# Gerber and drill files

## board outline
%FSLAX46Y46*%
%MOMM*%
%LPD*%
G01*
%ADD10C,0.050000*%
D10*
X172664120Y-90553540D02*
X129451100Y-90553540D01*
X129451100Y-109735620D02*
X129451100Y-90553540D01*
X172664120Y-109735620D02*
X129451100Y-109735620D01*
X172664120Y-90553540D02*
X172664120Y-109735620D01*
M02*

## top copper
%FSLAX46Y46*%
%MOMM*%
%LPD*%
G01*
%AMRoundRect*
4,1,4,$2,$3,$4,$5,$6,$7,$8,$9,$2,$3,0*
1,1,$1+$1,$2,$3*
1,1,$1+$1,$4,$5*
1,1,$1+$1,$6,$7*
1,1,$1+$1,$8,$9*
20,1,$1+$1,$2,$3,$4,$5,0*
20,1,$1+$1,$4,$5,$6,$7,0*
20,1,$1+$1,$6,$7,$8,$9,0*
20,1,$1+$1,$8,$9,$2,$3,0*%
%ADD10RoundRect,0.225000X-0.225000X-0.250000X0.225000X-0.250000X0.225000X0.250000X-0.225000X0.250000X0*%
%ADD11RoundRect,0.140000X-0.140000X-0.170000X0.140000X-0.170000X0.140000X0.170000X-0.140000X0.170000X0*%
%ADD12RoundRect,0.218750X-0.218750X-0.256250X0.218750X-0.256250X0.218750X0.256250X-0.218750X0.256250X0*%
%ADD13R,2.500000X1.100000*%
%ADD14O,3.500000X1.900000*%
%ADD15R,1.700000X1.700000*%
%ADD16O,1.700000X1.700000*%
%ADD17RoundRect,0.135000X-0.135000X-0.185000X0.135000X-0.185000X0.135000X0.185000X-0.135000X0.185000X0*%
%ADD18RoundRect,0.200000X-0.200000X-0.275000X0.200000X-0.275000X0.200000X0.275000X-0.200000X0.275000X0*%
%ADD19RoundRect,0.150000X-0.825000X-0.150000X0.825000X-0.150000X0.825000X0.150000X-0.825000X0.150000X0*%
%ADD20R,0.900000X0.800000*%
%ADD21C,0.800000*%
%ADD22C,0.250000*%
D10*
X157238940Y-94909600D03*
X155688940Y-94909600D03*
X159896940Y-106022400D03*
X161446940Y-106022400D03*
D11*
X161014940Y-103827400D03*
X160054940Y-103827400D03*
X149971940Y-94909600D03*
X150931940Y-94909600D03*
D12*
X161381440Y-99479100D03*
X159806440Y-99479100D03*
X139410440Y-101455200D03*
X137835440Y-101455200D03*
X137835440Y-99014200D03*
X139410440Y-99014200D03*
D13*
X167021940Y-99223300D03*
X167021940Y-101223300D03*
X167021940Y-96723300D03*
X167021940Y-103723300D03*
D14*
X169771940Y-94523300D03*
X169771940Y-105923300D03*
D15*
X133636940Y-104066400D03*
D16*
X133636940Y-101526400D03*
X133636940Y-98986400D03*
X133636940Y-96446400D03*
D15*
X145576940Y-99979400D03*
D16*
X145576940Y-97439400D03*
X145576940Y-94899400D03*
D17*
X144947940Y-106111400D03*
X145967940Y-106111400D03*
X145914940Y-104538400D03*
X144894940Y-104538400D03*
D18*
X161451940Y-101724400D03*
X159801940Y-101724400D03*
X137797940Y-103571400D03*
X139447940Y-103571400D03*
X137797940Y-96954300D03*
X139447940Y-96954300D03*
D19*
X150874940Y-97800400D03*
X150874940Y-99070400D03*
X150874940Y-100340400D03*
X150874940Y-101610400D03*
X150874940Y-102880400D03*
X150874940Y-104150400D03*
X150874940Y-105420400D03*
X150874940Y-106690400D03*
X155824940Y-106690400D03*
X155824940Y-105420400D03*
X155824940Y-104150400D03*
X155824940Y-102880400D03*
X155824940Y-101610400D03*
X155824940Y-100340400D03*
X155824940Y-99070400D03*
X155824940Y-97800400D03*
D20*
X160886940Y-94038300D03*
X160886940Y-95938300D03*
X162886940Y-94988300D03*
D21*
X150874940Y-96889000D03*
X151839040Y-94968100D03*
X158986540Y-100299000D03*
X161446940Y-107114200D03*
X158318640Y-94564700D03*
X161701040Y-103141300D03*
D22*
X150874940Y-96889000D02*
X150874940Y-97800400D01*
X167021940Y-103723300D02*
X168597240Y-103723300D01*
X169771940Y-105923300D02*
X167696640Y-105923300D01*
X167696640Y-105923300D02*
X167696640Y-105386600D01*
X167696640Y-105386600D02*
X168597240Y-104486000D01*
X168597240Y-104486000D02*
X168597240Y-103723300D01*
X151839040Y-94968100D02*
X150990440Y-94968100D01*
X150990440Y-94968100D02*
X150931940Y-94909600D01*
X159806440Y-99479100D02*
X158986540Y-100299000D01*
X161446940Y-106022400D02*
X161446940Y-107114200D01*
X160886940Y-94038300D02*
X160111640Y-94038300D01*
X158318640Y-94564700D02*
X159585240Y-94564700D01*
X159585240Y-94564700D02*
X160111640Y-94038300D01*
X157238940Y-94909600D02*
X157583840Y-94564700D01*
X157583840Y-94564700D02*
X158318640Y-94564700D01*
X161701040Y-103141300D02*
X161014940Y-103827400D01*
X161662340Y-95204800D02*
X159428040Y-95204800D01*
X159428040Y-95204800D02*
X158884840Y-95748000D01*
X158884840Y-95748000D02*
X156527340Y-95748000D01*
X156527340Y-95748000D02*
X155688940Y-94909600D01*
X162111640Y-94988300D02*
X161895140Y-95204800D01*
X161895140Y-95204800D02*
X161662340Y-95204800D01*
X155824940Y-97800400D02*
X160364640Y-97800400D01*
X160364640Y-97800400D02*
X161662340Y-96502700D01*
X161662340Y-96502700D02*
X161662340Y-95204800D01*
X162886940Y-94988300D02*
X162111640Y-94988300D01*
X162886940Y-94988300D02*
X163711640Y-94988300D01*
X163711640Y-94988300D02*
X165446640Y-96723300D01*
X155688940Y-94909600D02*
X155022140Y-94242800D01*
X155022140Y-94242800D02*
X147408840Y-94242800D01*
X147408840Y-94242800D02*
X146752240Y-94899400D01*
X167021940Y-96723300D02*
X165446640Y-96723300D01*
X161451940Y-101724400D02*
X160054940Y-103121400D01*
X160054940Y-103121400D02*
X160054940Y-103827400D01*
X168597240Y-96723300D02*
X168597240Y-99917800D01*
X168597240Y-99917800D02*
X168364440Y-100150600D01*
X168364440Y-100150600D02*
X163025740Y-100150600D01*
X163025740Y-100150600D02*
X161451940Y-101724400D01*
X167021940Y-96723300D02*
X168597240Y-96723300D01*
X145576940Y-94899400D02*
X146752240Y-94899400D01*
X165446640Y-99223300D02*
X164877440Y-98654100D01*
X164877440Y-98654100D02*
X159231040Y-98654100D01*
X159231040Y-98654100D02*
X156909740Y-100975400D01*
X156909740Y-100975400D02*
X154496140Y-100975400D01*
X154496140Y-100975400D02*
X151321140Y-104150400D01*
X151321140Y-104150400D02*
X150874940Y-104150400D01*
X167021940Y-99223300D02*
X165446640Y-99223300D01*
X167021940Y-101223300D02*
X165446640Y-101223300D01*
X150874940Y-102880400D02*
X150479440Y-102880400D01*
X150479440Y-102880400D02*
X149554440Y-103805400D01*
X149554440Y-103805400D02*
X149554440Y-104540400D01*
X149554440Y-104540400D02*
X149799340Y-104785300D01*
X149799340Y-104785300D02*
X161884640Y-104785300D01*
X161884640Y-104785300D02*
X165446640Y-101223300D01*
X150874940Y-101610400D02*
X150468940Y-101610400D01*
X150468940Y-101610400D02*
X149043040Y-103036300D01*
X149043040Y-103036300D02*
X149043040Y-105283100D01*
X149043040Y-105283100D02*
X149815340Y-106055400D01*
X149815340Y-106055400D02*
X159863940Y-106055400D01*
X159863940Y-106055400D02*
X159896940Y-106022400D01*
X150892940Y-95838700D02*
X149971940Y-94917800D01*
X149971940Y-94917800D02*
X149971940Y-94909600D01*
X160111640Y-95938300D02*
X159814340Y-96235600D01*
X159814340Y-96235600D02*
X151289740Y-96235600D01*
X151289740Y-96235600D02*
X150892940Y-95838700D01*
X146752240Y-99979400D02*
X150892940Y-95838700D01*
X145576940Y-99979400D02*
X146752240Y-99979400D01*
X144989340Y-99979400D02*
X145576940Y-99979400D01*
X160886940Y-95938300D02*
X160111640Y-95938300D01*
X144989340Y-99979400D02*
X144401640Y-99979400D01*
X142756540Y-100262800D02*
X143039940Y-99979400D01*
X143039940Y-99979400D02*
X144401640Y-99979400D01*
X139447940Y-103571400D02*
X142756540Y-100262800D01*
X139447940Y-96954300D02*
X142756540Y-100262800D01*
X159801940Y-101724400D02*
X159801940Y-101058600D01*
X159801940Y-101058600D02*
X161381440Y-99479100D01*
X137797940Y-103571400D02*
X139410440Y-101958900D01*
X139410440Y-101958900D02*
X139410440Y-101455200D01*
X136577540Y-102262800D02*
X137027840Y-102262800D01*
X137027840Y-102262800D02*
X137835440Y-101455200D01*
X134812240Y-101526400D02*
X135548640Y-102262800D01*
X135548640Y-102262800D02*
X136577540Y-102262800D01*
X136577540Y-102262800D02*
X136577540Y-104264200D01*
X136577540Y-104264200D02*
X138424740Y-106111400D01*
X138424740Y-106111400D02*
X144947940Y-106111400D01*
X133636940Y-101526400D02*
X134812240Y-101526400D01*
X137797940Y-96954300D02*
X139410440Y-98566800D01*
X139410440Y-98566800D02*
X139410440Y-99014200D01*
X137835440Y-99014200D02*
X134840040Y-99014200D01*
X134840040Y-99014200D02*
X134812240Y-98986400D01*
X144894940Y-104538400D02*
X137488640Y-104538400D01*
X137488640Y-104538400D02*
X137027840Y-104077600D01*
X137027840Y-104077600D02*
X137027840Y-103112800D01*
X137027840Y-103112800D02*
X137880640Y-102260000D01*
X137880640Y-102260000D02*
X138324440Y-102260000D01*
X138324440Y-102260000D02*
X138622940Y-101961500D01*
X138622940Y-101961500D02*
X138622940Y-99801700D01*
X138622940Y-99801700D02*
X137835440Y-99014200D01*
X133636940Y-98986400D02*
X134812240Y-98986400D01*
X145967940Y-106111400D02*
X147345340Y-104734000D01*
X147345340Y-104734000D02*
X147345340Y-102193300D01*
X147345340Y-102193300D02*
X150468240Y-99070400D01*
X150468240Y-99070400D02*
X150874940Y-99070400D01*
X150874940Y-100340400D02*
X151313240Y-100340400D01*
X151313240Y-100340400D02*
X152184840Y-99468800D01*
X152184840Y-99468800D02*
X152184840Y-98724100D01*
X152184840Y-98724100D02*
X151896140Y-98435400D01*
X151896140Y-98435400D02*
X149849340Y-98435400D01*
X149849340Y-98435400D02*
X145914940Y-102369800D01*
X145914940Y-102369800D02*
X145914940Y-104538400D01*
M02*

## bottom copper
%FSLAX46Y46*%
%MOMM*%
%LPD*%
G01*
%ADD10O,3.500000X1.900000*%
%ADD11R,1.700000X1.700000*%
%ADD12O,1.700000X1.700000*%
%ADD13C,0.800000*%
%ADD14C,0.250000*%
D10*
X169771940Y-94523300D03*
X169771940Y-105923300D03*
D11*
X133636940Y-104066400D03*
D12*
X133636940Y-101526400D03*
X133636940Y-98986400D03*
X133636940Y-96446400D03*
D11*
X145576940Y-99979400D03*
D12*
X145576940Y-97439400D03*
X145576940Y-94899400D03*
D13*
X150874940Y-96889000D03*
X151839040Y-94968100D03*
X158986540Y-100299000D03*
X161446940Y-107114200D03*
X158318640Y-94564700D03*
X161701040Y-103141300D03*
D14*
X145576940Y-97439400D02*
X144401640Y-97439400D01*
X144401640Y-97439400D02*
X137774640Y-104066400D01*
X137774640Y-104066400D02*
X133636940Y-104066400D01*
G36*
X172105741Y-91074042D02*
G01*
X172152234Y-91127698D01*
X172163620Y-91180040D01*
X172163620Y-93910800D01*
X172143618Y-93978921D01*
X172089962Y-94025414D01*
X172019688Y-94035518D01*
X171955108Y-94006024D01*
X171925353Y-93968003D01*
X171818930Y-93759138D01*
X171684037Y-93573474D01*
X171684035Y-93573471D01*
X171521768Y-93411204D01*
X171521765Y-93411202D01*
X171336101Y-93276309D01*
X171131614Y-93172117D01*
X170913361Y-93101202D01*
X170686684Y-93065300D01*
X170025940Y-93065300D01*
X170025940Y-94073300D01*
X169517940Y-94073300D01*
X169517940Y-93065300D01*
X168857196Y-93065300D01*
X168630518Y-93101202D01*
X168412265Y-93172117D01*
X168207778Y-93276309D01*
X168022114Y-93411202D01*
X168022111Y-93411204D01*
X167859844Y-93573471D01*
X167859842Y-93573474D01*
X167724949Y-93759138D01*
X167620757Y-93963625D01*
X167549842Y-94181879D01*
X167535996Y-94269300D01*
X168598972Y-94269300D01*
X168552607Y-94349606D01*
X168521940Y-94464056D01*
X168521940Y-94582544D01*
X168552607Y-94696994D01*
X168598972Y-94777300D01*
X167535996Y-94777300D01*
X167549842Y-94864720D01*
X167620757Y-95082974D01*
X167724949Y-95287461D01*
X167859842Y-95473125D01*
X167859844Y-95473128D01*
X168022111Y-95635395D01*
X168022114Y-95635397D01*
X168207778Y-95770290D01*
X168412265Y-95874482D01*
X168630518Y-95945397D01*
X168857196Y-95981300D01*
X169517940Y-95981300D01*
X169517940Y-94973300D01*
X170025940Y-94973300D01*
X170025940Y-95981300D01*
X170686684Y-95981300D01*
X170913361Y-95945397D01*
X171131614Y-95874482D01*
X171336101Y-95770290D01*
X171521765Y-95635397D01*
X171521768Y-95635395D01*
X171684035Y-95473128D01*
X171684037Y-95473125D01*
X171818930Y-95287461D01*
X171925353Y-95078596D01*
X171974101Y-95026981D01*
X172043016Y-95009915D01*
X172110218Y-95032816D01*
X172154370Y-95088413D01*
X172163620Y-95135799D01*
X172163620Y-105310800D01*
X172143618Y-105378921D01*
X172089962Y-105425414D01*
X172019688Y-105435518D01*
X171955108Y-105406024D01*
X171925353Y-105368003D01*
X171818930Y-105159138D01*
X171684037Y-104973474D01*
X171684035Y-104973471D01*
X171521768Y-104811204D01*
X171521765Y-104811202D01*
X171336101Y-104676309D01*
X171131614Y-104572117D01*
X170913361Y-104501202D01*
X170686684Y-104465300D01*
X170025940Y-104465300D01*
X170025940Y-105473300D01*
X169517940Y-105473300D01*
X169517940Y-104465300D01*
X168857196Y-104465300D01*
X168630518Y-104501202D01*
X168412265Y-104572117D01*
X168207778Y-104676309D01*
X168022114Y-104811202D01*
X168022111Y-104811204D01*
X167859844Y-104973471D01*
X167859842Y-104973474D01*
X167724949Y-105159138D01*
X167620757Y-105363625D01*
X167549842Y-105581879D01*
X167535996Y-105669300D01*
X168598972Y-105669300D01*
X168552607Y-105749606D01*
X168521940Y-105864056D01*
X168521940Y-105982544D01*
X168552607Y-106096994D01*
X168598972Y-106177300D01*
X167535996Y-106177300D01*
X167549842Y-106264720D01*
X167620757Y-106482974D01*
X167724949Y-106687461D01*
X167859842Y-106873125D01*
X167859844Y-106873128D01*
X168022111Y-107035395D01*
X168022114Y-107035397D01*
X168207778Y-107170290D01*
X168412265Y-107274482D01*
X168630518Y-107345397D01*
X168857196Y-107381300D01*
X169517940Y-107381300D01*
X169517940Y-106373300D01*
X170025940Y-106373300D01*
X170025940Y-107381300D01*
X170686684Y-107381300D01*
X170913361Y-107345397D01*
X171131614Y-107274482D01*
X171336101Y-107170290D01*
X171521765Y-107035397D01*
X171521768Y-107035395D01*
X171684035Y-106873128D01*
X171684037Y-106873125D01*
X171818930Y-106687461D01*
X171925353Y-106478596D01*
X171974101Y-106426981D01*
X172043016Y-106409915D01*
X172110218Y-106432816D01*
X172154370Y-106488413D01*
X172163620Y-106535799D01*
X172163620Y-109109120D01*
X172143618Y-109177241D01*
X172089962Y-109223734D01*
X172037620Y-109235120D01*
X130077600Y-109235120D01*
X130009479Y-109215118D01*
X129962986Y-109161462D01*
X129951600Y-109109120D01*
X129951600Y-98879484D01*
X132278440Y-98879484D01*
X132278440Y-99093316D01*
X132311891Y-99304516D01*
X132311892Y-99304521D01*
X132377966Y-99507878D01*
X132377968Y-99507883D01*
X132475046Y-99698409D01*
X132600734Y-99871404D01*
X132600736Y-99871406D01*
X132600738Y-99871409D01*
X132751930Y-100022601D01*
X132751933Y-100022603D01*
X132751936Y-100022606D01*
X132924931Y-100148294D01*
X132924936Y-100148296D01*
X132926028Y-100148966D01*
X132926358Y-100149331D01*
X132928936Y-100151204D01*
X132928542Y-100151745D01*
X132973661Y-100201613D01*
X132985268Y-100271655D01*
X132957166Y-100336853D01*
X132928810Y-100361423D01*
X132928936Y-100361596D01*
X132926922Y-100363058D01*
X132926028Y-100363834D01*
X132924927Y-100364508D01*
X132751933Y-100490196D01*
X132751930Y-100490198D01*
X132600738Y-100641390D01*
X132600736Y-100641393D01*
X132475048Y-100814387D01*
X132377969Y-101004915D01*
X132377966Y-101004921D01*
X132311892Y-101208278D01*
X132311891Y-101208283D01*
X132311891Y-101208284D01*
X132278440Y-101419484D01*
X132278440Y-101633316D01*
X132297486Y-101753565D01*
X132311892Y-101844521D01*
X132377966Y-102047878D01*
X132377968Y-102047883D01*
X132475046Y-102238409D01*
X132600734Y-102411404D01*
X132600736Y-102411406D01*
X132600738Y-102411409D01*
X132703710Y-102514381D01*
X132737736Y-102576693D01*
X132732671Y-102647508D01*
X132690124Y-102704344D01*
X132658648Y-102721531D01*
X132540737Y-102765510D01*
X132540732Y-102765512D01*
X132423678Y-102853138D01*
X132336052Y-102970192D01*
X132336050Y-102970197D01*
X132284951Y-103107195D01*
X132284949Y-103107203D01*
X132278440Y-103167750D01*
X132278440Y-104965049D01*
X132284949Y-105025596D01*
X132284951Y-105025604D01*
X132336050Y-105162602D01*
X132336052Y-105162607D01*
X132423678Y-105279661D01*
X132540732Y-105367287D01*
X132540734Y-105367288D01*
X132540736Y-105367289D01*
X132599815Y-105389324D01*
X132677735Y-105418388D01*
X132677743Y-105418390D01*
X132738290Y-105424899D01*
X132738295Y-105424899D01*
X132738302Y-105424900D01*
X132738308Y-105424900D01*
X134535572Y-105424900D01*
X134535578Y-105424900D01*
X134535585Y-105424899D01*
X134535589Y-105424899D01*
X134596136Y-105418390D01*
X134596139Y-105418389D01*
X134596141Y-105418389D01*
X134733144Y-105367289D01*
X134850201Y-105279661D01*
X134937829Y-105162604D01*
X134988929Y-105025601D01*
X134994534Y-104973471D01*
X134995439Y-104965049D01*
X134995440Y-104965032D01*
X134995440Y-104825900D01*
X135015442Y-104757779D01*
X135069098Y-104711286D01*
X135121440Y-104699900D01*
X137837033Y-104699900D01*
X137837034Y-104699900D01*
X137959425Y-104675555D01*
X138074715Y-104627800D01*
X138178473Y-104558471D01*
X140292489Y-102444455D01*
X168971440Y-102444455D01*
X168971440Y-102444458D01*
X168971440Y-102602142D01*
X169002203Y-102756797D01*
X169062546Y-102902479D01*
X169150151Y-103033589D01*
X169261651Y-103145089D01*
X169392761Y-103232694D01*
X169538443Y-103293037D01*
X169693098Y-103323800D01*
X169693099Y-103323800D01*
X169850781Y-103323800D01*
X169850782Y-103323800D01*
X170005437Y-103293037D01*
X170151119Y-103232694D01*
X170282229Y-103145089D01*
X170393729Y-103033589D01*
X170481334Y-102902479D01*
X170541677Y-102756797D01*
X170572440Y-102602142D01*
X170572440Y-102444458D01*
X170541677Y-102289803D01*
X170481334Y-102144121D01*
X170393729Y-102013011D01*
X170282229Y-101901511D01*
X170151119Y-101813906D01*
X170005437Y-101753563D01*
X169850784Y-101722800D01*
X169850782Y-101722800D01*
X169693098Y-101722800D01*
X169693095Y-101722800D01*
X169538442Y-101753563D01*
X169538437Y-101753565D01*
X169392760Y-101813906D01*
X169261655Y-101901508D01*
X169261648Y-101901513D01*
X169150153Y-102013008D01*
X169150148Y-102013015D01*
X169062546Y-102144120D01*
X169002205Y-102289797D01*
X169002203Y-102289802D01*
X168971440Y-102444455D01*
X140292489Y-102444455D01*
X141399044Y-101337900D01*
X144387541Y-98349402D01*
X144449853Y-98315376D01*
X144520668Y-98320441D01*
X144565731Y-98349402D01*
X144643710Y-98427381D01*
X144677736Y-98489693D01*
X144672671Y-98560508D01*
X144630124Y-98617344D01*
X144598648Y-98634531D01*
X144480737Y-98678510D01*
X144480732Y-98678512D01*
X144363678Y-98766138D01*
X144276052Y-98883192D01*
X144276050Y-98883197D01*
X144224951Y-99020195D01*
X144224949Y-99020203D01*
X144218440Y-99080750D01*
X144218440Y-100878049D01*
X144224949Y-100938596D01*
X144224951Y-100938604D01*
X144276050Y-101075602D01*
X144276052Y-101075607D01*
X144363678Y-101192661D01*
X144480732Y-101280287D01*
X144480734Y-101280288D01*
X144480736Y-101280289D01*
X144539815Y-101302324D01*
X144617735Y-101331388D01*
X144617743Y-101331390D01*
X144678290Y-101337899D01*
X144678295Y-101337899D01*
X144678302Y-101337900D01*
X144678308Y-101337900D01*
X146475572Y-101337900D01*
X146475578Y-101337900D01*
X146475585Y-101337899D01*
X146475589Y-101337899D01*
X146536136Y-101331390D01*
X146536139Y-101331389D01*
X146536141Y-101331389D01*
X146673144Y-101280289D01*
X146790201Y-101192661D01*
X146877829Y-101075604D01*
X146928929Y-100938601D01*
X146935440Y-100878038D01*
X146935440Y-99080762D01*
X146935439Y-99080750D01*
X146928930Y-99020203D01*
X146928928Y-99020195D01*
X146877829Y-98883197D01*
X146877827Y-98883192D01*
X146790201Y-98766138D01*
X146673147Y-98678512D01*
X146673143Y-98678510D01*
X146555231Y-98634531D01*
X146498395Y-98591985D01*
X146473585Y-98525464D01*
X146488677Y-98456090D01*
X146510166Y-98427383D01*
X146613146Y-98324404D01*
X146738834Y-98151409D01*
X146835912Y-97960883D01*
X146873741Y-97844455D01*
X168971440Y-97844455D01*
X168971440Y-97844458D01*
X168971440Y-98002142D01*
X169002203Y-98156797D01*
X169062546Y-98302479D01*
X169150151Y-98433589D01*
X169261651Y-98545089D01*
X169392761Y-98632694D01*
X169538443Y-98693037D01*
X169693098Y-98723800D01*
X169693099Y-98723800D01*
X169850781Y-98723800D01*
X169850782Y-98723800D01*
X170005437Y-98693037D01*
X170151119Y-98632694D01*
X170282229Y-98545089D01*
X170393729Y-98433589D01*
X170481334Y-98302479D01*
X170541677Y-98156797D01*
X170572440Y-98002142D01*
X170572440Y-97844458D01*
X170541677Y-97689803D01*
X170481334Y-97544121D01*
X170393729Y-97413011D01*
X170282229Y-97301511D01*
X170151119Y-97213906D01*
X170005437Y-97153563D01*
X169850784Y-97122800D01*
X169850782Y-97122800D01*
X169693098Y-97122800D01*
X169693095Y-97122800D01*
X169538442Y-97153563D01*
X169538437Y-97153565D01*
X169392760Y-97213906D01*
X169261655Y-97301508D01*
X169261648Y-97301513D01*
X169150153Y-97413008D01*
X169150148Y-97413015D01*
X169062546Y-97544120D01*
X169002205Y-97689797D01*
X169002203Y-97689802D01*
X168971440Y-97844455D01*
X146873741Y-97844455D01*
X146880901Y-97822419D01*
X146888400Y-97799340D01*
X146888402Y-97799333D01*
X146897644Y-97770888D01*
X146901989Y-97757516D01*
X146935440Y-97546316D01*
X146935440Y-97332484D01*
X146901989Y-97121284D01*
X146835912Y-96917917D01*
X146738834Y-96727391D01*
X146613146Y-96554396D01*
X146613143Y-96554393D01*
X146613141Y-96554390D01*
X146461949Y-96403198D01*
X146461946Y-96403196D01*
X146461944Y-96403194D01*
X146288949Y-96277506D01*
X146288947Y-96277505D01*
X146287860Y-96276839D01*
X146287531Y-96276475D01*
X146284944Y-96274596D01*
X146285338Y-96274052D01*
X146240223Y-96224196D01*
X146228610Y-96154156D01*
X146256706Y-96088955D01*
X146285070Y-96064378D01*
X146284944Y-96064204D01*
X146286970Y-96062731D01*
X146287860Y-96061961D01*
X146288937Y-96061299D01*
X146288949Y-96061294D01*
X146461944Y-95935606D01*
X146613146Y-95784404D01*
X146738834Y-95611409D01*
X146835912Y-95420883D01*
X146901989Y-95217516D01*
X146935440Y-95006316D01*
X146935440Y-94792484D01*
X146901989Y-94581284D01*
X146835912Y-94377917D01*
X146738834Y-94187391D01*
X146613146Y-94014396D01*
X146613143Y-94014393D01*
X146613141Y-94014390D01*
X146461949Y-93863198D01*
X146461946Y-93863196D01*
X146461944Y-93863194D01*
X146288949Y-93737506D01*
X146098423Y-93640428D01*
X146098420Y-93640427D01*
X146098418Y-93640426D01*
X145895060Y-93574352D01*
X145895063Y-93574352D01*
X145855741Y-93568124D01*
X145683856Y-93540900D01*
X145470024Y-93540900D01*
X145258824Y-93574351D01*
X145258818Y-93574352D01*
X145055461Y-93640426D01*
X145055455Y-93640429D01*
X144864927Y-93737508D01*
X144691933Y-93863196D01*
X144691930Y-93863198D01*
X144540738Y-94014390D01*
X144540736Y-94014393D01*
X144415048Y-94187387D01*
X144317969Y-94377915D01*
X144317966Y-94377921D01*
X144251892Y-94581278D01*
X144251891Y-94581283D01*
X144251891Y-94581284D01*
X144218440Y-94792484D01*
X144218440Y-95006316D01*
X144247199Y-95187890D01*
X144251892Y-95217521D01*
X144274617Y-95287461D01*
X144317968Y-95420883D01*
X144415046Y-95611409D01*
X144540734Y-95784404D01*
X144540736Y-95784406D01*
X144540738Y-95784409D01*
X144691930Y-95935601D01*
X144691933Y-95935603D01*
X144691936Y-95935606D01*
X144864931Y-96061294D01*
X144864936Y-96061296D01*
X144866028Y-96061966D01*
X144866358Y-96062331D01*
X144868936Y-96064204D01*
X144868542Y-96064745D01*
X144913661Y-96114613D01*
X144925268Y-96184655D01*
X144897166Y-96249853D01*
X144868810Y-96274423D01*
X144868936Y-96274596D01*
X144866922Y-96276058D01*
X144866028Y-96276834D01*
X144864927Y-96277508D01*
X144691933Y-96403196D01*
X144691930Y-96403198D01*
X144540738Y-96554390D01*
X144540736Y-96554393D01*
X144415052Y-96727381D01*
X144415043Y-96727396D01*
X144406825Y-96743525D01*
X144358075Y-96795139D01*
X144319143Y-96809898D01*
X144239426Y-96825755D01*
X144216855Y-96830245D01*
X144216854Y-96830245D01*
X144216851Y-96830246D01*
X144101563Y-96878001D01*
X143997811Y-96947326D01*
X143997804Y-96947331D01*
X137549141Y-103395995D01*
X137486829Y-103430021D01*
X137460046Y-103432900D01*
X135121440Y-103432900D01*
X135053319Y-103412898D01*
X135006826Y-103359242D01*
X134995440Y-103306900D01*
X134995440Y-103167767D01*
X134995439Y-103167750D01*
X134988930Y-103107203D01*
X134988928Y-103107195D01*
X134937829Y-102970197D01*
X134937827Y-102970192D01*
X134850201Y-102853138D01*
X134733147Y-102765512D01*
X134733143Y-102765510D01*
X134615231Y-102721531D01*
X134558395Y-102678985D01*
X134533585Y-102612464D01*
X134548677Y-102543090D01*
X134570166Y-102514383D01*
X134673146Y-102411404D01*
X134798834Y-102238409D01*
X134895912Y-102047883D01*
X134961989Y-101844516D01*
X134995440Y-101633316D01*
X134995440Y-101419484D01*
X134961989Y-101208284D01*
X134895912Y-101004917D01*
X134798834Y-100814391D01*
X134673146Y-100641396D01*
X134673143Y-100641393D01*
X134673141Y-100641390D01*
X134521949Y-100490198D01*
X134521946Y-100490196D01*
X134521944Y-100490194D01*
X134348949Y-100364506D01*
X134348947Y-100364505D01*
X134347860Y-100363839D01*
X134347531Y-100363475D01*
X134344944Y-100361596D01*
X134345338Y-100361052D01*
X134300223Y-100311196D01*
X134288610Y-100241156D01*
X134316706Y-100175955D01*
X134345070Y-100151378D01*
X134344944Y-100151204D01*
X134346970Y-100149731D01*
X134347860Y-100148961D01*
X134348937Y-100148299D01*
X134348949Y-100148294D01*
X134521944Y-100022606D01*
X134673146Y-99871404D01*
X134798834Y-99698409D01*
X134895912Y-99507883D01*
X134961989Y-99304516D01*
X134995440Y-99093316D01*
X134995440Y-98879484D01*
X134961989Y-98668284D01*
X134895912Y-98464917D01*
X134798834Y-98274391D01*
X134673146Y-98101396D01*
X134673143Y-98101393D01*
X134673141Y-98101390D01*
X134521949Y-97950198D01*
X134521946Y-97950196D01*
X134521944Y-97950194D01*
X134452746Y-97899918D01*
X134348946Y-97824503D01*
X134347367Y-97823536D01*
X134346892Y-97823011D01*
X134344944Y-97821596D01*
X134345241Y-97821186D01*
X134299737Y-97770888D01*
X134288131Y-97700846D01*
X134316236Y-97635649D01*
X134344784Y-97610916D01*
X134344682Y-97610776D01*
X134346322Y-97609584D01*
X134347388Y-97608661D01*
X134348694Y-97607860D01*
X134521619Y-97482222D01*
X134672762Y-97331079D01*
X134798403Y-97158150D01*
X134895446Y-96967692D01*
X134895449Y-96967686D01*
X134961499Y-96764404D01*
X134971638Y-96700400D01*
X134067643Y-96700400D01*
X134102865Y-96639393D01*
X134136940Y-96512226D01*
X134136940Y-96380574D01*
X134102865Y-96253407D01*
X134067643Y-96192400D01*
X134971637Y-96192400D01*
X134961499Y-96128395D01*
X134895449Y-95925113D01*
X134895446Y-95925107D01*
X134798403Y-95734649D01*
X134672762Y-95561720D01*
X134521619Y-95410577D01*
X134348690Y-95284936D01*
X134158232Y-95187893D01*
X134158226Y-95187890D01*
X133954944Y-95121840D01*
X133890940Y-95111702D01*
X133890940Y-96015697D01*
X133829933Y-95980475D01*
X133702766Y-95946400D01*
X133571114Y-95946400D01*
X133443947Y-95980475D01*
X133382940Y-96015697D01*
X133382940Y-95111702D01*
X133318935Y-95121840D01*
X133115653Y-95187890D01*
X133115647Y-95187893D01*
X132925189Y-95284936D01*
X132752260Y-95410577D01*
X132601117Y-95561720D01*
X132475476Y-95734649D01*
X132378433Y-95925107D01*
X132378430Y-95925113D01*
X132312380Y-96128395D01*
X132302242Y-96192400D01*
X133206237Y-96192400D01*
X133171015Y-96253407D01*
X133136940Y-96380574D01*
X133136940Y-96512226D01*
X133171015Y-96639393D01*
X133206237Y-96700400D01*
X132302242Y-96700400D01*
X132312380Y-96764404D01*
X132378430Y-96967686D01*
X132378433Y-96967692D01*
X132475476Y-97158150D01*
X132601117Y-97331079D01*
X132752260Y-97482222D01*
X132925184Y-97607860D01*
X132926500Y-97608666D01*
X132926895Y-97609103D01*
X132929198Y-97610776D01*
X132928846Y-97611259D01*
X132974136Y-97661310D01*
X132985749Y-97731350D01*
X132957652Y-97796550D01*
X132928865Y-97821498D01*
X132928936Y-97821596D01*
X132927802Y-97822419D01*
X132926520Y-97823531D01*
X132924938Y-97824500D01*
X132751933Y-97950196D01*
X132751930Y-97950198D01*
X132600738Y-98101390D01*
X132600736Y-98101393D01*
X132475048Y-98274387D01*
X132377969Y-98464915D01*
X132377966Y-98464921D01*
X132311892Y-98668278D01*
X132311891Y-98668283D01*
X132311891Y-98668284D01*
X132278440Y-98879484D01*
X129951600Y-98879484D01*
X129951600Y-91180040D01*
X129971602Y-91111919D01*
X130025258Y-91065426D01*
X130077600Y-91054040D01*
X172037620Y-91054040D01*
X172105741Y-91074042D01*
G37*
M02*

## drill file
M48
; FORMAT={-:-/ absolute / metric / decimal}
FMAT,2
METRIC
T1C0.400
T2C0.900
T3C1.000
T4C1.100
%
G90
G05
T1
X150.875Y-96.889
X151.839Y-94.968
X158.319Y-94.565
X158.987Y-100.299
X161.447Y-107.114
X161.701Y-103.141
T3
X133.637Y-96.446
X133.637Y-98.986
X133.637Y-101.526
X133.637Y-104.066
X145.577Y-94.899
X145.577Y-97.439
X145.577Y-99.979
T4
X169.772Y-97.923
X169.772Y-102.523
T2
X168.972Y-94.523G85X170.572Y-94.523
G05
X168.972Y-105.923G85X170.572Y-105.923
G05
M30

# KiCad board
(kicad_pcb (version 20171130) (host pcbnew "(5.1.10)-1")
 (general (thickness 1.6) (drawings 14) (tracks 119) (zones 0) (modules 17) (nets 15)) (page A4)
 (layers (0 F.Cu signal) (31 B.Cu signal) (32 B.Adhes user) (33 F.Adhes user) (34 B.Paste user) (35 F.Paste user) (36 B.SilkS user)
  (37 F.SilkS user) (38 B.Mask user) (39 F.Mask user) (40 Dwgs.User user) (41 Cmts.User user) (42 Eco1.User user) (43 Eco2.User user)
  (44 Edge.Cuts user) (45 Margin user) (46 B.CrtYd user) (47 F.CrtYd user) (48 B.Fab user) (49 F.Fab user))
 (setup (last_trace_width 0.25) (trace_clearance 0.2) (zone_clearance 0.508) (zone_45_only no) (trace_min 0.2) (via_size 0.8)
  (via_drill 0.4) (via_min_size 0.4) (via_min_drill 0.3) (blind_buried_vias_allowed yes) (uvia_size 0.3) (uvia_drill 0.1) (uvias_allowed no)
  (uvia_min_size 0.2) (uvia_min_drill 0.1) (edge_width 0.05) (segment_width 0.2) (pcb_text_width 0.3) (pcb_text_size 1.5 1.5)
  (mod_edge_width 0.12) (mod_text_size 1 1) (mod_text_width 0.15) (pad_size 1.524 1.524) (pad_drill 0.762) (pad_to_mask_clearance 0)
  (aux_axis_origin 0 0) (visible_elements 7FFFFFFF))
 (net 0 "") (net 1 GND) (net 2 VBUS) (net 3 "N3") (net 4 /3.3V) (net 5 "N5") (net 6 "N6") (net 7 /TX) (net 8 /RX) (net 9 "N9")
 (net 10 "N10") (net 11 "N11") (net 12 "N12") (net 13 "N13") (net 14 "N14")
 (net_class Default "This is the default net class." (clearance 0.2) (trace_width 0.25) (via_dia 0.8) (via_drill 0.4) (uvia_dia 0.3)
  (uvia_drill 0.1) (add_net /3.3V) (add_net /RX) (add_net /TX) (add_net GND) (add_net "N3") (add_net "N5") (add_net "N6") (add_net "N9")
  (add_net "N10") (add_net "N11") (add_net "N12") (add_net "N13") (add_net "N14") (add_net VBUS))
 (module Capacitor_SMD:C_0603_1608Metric (layer F.Cu) (at 156.46394 94.9096)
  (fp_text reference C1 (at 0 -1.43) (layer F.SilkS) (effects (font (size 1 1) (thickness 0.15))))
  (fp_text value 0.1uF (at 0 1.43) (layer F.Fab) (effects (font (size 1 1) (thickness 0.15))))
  (pad 2 smd roundrect (at 0.775 0) (size 0.9 0.95) (layers F.Cu F.Paste F.Mask) (roundrect_rratio 0.25) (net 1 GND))
  (pad 1 smd roundrect (at -0.775 0) (size 0.9 0.95) (layers F.Cu F.Paste F.Mask) (roundrect_rratio 0.25) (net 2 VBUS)))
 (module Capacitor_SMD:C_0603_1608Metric (layer F.Cu) (at 160.67194 106.0224)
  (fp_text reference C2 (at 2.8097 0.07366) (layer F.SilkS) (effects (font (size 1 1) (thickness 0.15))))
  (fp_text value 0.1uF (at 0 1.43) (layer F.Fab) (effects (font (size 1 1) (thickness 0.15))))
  (pad 1 smd roundrect (at -0.775 0) (size 0.9 0.95) (layers F.Cu F.Paste F.Mask) (roundrect_rratio 0.25) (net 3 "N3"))
  (pad 2 smd roundrect (at 0.775 0) (size 0.9 0.95) (layers F.Cu F.Paste F.Mask) (roundrect_rratio 0.25) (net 1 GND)))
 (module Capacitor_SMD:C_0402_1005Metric (layer F.Cu) (at 160.53494 103.8274)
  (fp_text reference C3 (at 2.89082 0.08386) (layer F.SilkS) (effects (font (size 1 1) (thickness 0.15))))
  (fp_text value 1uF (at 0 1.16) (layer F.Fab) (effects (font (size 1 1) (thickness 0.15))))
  (pad 2 smd roundrect (at 0.48 0) (size 0.56 0.62) (layers F.Cu F.Paste F.Mask) (roundrect_rratio 0.25) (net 1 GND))
  (pad 1 smd roundrect (at -0.48 0) (size 0.56 0.62) (layers F.Cu F.Paste F.Mask) (roundrect_rratio 0.25) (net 2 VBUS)))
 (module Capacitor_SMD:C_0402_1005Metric (layer F.Cu) (at 150.45194 94.9096)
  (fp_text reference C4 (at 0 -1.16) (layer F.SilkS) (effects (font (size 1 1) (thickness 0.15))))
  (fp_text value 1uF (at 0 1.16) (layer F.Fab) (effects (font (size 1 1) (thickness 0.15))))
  (pad 1 smd roundrect (at -0.48 0) (size 0.56 0.62) (layers F.Cu F.Paste F.Mask) (roundrect_rratio 0.25) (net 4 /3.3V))
  (pad 2 smd roundrect (at 0.48 0) (size 0.56 0.62) (layers F.Cu F.Paste F.Mask) (roundrect_rratio 0.25) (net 1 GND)))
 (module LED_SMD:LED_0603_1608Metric (layer F.Cu) (at 160.59394 99.4791)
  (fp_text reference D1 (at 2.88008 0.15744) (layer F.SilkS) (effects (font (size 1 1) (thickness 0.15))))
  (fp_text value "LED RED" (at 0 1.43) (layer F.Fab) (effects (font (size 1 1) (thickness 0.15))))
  (pad 2 smd roundrect (at 0.7875 0) (size 0.875 0.95) (layers F.Cu F.Paste F.Mask) (roundrect_rratio 0.25) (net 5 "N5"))
  (pad 1 smd roundrect (at -0.7875 0) (size 0.875 0.95) (layers F.Cu F.Paste F.Mask) (roundrect_rratio 0.25) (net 1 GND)))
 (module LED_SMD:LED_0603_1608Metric (layer F.Cu) (at 138.62294 101.4552)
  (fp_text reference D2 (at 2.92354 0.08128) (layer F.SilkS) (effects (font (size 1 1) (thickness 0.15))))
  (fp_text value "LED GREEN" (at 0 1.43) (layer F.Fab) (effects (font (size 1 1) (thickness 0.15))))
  (pad 2 smd roundrect (at 0.7875 0) (size 0.875 0.95) (layers F.Cu F.Paste F.Mask) (roundrect_rratio 0.25) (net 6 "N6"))
  (pad 1 smd roundrect (at -0.7875 0) (size 0.875 0.95) (layers F.Cu F.Paste F.Mask) (roundrect_rratio 0.25) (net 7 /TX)))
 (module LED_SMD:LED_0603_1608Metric (layer F.Cu) (at 138.62294 99.0142)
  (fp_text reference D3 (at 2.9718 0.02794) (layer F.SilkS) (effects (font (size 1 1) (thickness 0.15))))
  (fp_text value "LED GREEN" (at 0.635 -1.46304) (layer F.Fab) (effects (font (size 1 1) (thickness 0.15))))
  (pad 1 smd roundrect (at -0.7875 0) (size 0.875 0.95) (layers F.Cu F.Paste F.Mask) (roundrect_rratio 0.25) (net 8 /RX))
  (pad 2 smd roundrect (at 0.7875 0) (size 0.875 0.95) (layers F.Cu F.Paste F.Mask) (roundrect_rratio 0.25) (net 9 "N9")))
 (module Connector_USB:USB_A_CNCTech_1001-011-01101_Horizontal (layer F.Cu) (at 176.67194 100.2233)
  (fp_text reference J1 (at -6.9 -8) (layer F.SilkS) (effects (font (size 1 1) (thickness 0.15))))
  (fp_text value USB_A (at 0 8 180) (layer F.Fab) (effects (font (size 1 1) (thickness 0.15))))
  (pad 2 smd rect (at -9.65 -1) (size 2.5 1.1) (layers F.Cu F.Paste F.Mask) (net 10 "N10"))
  (pad 3 smd rect (at -9.65 1) (size 2.5 1.1) (layers F.Cu F.Paste F.Mask) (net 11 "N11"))
  (pad 1 smd rect (at -9.65 -3.5) (size 2.5 1.1) (layers F.Cu F.Paste F.Mask) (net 2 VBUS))
  (pad 4 smd rect (at -9.65 3.5) (size 2.5 1.1) (layers F.Cu F.Paste F.Mask) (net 1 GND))
  (pad 5 thru_hole oval (at -6.9 -5.7) (size 3.5 1.9) (drill oval 2.5 0.9) (layers *.Cu *.Mask) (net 1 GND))
  (pad 5 thru_hole oval (at -6.9 5.7) (size 3.5 1.9) (drill oval 2.5 0.9) (layers *.Cu *.Mask) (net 1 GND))
  (pad "" np_thru_hole circle (at -6.9 -2.3) (size 1.1 1.1) (drill 1.1) (layers *.Cu *.Mask))
  (pad "" np_thru_hole circle (at -6.9 2.3) (size 1.1 1.1) (drill 1.1) (layers *.Cu *.Mask)))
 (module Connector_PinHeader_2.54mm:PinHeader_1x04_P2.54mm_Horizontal (layer F.Cu) (at 133.63694 104.0664 180)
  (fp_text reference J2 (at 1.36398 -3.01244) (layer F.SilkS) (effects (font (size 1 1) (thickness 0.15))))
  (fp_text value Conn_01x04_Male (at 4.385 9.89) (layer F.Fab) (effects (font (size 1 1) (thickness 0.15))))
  (pad 1 thru_hole rect (at 0 0 180) (size 1.7 1.7) (drill 1) (layers *.Cu *.Mask) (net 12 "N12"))
  (pad 2 thru_hole oval (at 0 2.54 180) (size 1.7 1.7) (drill 1) (layers *.Cu *.Mask) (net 7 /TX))
  (pad 3 thru_hole oval (at 0 5.08 180) (size 1.7 1.7) (drill 1) (layers *.Cu *.Mask) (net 8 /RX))
  (pad 4 thru_hole oval (at 0 7.62 180) (size 1.7 1.7) (drill 1) (layers *.Cu *.Mask) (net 1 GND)))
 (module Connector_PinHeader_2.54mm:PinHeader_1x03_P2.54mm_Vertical (layer F.Cu) (at 145.57694 99.9794 180)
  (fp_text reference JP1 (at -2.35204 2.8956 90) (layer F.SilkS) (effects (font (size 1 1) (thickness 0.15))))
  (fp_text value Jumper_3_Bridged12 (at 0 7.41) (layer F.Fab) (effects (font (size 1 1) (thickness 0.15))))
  (pad 1 thru_hole rect (at 0 0 180) (size 1.7 1.7) (drill 1) (layers *.Cu *.Mask) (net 4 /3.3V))
  (pad 2 thru_hole oval (at 0 2.54 180) (size 1.7 1.7) (drill 1) (layers *.Cu *.Mask) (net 12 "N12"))
  (pad 3 thru_hole oval (at 0 5.08 180) (size 1.7 1.7) (drill 1) (layers *.Cu *.Mask) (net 2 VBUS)))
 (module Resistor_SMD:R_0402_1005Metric (layer F.Cu) (at 145.45794 106.1114)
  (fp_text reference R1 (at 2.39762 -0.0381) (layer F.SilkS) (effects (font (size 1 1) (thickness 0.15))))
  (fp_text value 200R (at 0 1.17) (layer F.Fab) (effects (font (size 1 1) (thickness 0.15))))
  (pad 1 smd roundrect (at -0.51 0) (size 0.54 0.64) (layers F.Cu F.Paste F.Mask) (roundrect_rratio 0.25) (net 7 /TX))
  (pad 2 smd roundrect (at 0.51 0) (size 0.54 0.64) (layers F.Cu F.Paste F.Mask) (roundrect_rratio 0.25) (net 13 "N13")))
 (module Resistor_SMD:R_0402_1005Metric (layer F.Cu) (at 145.40494 104.5384)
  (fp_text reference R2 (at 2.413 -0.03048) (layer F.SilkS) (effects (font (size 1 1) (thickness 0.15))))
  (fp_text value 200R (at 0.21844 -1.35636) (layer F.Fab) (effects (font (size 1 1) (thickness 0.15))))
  (pad 2 smd roundrect (at 0.51 0) (size 0.54 0.64) (layers F.Cu F.Paste F.Mask) (roundrect_rratio 0.25) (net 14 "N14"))
  (pad 1 smd roundrect (at -0.51 0) (size 0.54 0.64) (layers F.Cu F.Paste F.Mask) (roundrect_rratio 0.25) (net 8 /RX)))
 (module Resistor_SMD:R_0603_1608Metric (layer F.Cu) (at 160.62694 101.7244)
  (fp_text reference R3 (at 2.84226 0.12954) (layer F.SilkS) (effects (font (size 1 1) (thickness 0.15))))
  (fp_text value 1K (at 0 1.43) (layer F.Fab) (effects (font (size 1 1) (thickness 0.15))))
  (pad 2 smd roundrect (at 0.825 0) (size 0.8 0.95) (layers F.Cu F.Paste F.Mask) (roundrect_rratio 0.25) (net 2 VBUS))
  (pad 1 smd roundrect (at -0.825 0) (size 0.8 0.95) (layers F.Cu F.Paste F.Mask) (roundrect_rratio 0.25) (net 5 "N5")))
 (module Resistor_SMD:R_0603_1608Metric (layer F.Cu) (at 138.62294 103.5714)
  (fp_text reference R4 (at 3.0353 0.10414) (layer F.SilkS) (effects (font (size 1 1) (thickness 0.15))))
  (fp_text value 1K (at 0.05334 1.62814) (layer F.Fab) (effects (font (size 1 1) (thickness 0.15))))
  (pad 1 smd roundrect (at -0.825 0) (size 0.8 0.95) (layers F.Cu F.Paste F.Mask) (roundrect_rratio 0.25) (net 6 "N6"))
  (pad 2 smd roundrect (at 0.825 0) (size 0.8 0.95) (layers F.Cu F.Paste F.Mask) (roundrect_rratio 0.25) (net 4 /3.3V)))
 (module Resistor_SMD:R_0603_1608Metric (layer F.Cu) (at 138.62294 96.9543)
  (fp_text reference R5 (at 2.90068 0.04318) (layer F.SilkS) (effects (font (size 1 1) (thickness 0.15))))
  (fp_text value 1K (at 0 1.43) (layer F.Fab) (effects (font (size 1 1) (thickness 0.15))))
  (pad 1 smd roundrect (at -0.825 0) (size 0.8 0.95) (layers F.Cu F.Paste F.Mask) (roundrect_rratio 0.25) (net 9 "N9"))
  (pad 2 smd roundrect (at 0.825 0) (size 0.8 0.95) (layers F.Cu F.Paste F.Mask) (roundrect_rratio 0.25) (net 4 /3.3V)))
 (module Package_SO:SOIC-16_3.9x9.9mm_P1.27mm (layer F.Cu) (at 153.34994 102.2454)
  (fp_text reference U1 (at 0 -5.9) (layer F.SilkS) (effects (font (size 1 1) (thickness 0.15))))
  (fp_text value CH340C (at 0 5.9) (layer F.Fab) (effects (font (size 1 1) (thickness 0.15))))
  (pad 1 smd roundrect (at -2.475 -4.445) (size 1.95 0.6) (layers F.Cu F.Paste F.Mask) (roundrect_rratio 0.25) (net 1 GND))
  (pad 2 smd roundrect (at -2.475 -3.175) (size 1.95 0.6) (layers F.Cu F.Paste F.Mask) (roundrect_rratio 0.25) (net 13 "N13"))
  (pad 3 smd roundrect (at -2.475 -1.905) (size 1.95 0.6) (layers F.Cu F.Paste F.Mask) (roundrect_rratio 0.25) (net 14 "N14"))
  (pad 4 smd roundrect (at -2.475 -0.635) (size 1.95 0.6) (layers F.Cu F.Paste F.Mask) (roundrect_rratio 0.25) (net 3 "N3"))
  (pad 5 smd roundrect (at -2.475 0.635) (size 1.95 0.6) (layers F.Cu F.Paste F.Mask) (roundrect_rratio 0.25) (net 11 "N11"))
  (pad 6 smd roundrect (at -2.475 1.905) (size 1.95 0.6) (layers F.Cu F.Paste F.Mask) (roundrect_rratio 0.25) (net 10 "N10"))
  (pad 7 smd roundrect (at -2.475 3.175) (size 1.95 0.6) (layers F.Cu F.Paste F.Mask) (roundrect_rratio 0.25))
  (pad 8 smd roundrect (at -2.475 4.445) (size 1.95 0.6) (layers F.Cu F.Paste F.Mask) (roundrect_rratio 0.25))
  (pad 9 smd roundrect (at 2.475 4.445) (size 1.95 0.6) (layers F.Cu F.Paste F.Mask) (roundrect_rratio 0.25))
  (pad 10 smd roundrect (at 2.475 3.175) (size 1.95 0.6) (layers F.Cu F.Paste F.Mask) (roundrect_rratio 0.25))
  (pad 11 smd roundrect (at 2.475 1.905) (size 1.95 0.6) (layers F.Cu F.Paste F.Mask) (roundrect_rratio 0.25))
  (pad 12 smd roundrect (at 2.475 0.635) (size 1.95 0.6) (layers F.Cu F.Paste F.Mask) (roundrect_rratio 0.25))
  (pad 13 smd roundrect (at 2.475 -0.635) (size 1.95 0.6) (layers F.Cu F.Paste F.Mask) (roundrect_rratio 0.25))
  (pad 14 smd roundrect (at 2.475 -1.905) (size 1.95 0.6) (layers F.Cu F.Paste F.Mask) (roundrect_rratio 0.25))
  (pad 15 smd roundrect (at 2.475 -3.175) (size 1.95 0.6) (layers F.Cu F.Paste F.Mask) (roundrect_rratio 0.25))
  (pad 16 smd roundrect (at 2.475 -4.445) (size 1.95 0.6) (layers F.Cu F.Paste F.Mask) (roundrect_rratio 0.25) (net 2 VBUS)))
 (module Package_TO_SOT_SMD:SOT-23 (layer F.Cu) (at 161.88694 94.9883)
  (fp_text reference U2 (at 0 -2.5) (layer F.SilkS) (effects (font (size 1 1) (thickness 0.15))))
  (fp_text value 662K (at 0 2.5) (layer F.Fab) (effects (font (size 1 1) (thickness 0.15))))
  (pad 1 smd rect (at -1 -0.95) (size 0.9 0.8) (layers F.Cu F.Paste F.Mask) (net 1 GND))
  (pad 2 smd rect (at -1 0.95) (size 0.9 0.8) (layers F.Cu F.Paste F.Mask) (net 4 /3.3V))
  (pad 3 smd rect (at 1 0) (size 0.9 0.8) (layers F.Cu F.Paste F.Mask) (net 2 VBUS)))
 (gr_line (start 172.66412 90.55354) (end 129.4511 90.55354) (layer Edge.Cuts) (width 0.05))
 (gr_line (start 129.4511 109.73562) (end 129.4511 90.55354) (layer Edge.Cuts) (width 0.05))
 (gr_line (start 172.66412 109.73562) (end 129.4511 109.73562) (layer Edge.Cuts) (width 0.05))
 (gr_line (start 172.66412 90.55354) (end 172.66412 109.73562) (layer Edge.Cuts) (width 0.05))
 (segment (start 150.87494 96.889) (end 150.87494 97.8004) (width 0.25) (layer F.Cu) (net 1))
 (segment (start 167.02194 103.7233) (end 168.59724 103.7233) (width 0.25) (layer F.Cu) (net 1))
 (segment (start 169.77194 105.9233) (end 167.69664 105.9233) (width 0.25) (layer F.Cu) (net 1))
 (segment (start 167.69664 105.9233) (end 167.69664 105.3866) (width 0.25) (layer F.Cu) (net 1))
 (segment (start 167.69664 105.3866) (end 168.59724 104.486) (width 0.25) (layer F.Cu) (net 1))
 (segment (start 168.59724 104.486) (end 168.59724 103.7233) (width 0.25) (layer F.Cu) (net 1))
 (segment (start 151.83904 94.9681) (end 150.99044 94.9681) (width 0.25) (layer F.Cu) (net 1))
 (segment (start 150.99044 94.9681) (end 150.93194 94.9096) (width 0.25) (layer F.Cu) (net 1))
 (segment (start 159.80644 99.4791) (end 158.98654 100.299) (width 0.25) (layer F.Cu) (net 1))
 (segment (start 161.44694 106.0224) (end 161.44694 107.1142) (width 0.25) (layer F.Cu) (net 1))
 (segment (start 160.88694 94.0383) (end 160.11164 94.0383) (width 0.25) (layer F.Cu) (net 1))
 (segment (start 158.31864 94.5647) (end 159.58524 94.5647) (width 0.25) (layer F.Cu) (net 1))
 (segment (start 159.58524 94.5647) (end 160.11164 94.0383) (width 0.25) (layer F.Cu) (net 1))
 (segment (start 157.23894 94.9096) (end 157.58384 94.5647) (width 0.25) (layer F.Cu) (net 1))
 (segment (start 157.58384 94.5647) (end 158.31864 94.5647) (width 0.25) (layer F.Cu) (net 1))
 (segment (start 161.70104 103.1413) (end 161.01494 103.8274) (width 0.25) (layer F.Cu) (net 1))
 (via (at 150.87494 96.889) (size 0.8) (layers F.Cu B.Cu) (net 1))
 (via (at 151.83904 94.9681) (size 0.8) (layers F.Cu B.Cu) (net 1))
 (via (at 158.98654 100.299) (size 0.8) (layers F.Cu B.Cu) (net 1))
 (via (at 161.44694 107.1142) (size 0.8) (layers F.Cu B.Cu) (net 1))
 (via (at 158.31864 94.5647) (size 0.8) (layers F.Cu B.Cu) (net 1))
 (via (at 161.70104 103.1413) (size 0.8) (layers F.Cu B.Cu) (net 1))
 (segment (start 161.66234 95.2048) (end 159.42804 95.2048) (width 0.25) (layer F.Cu) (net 2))
 (segment (start 159.42804 95.2048) (end 158.88484 95.748) (width 0.25) (layer F.Cu) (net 2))
 (segment (start 158.88484 95.748) (end 156.52734 95.748) (width 0.25) (layer F.Cu) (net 2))
 (segment (start 156.52734 95.748) (end 155.68894 94.9096) (width 0.25) (layer F.Cu) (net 2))
 (segment (start 162.11164 94.9883) (end 161.89514 95.2048) (width 0.25) (layer F.Cu) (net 2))
 (segment (start 161.89514 95.2048) (end 161.66234 95.2048) (width 0.25) (layer F.Cu) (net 2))
 (segment (start 155.82494 97.8004) (end 160.36464 97.8004) (width 0.25) (layer F.Cu) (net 2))
 (segment (start 160.36464 97.8004) (end 161.66234 96.5027) (width 0.25) (layer F.Cu) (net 2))
 (segment (start 161.66234 96.5027) (end 161.66234 95.2048) (width 0.25) (layer F.Cu) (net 2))
 (segment (start 162.88694 94.9883) (end 162.11164 94.9883) (width 0.25) (layer F.Cu) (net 2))
 (segment (start 162.88694 94.9883) (end 163.71164 94.9883) (width 0.25) (layer F.Cu) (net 2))
 (segment (start 163.71164 94.9883) (end 165.44664 96.7233) (width 0.25) (layer F.Cu) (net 2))
 (segment (start 155.68894 94.9096) (end 155.02214 94.2428) (width 0.25) (layer F.Cu) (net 2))
 (segment (start 155.02214 94.2428) (end 147.40884 94.2428) (width 0.25) (layer F.Cu) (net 2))
 (segment (start 147.40884 94.2428) (end 146.75224 94.8994) (width 0.25) (layer F.Cu) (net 2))
 (segment (start 167.02194 96.7233) (end 165.44664 96.7233) (width 0.25) (layer F.Cu) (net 2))
 (segment (start 161.45194 101.7244) (end 160.05494 103.1214) (width 0.25) (layer F.Cu) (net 2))
 (segment (start 160.05494 103.1214) (end 160.05494 103.8274) (width 0.25) (layer F.Cu) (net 2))
 (segment (start 168.59724 96.7233) (end 168.59724 99.9178) (width 0.25) (layer F.Cu) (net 2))
 (segment (start 168.59724 99.9178) (end 168.36444 100.1506) (width 0.25) (layer F.Cu) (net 2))
 (segment (start 168.36444 100.1506) (end 163.02574 100.1506) (width 0.25) (layer F.Cu) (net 2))
 (segment (start 163.02574 100.1506) (end 161.45194 101.7244) (width 0.25) (layer F.Cu) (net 2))
 (segment (start 167.02194 96.7233) (end 168.59724 96.7233) (width 0.25) (layer F.Cu) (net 2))
 (segment (start 145.57694 94.8994) (end 146.75224 94.8994) (width 0.25) (layer F.Cu) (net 2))
 (segment (start 165.44664 99.2233) (end 164.87744 98.6541) (width 0.25) (layer F.Cu) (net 10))
 (segment (start 164.87744 98.6541) (end 159.23104 98.6541) (width 0.25) (layer F.Cu) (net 10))
 (segment (start 159.23104 98.6541) (end 156.90974 100.9754) (width 0.25) (layer F.Cu) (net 10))
 (segment (start 156.90974 100.9754) (end 154.49614 100.9754) (width 0.25) (layer F.Cu) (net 10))
 (segment (start 154.49614 100.9754) (end 151.32114 104.1504) (width 0.25) (layer F.Cu) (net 10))
 (segment (start 151.32114 104.1504) (end 150.87494 104.1504) (width 0.25) (layer F.Cu) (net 10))
 (segment (start 167.02194 99.2233) (end 165.44664 99.2233) (width 0.25) (layer F.Cu) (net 10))
 (segment (start 167.02194 101.2233) (end 165.44664 101.2233) (width 0.25) (layer F.Cu) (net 11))
 (segment (start 150.87494 102.8804) (end 150.47944 102.8804) (width 0.25) (layer F.Cu) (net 11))
 (segment (start 150.47944 102.8804) (end 149.55444 103.8054) (width 0.25) (layer F.Cu) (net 11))
 (segment (start 149.55444 103.8054) (end 149.55444 104.5404) (width 0.25) (layer F.Cu) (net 11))
 (segment (start 149.55444 104.5404) (end 149.79934 104.7853) (width 0.25) (layer F.Cu) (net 11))
 (segment (start 149.79934 104.7853) (end 161.88464 104.7853) (width 0.25) (layer F.Cu) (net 11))
 (segment (start 161.88464 104.7853) (end 165.44664 101.2233) (width 0.25) (layer F.Cu) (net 11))
 (segment (start 150.87494 101.6104) (end 150.46894 101.6104) (width 0.25) (layer F.Cu) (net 3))
 (segment (start 150.46894 101.6104) (end 149.04304 103.0363) (width 0.25) (layer F.Cu) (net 3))
 (segment (start 149.04304 103.0363) (end 149.04304 105.2831) (width 0.25) (layer F.Cu) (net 3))
 (segment (start 149.04304 105.2831) (end 149.81534 106.0554) (width 0.25) (layer F.Cu) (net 3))
 (segment (start 149.81534 106.0554) (end 159.86394 106.0554) (width 0.25) (layer F.Cu) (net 3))
 (segment (start 159.86394 106.0554) (end 159.89694 106.0224) (width 0.25) (layer F.Cu) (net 3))
 (segment (start 150.89294 95.8387) (end 149.97194 94.9178) (width 0.25) (layer F.Cu) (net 4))
 (segment (start 149.97194 94.9178) (end 149.97194 94.9096) (width 0.25) (layer F.Cu) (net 4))
 (segment (start 160.11164 95.9383) (end 159.81434 96.2356) (width 0.25) (layer F.Cu) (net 4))
 (segment (start 159.81434 96.2356) (end 151.28974 96.2356) (width 0.25) (layer F.Cu) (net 4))
 (segment (start 151.28974 96.2356) (end 150.89294 95.8387) (width 0.25) (layer F.Cu) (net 4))
 (segment (start 146.75224 99.9794) (end 150.89294 95.8387) (width 0.25) (layer F.Cu) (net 4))
 (segment (start 145.57694 99.9794) (end 146.75224 99.9794) (width 0.25) (layer F.Cu) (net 4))
 (segment (start 144.98934 99.9794) (end 145.57694 99.9794) (width 0.25) (layer F.Cu) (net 4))
 (segment (start 160.88694 95.9383) (end 160.11164 95.9383) (width 0.25) (layer F.Cu) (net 4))
 (segment (start 144.98934 99.9794) (end 144.40164 99.9794) (width 0.25) (layer F.Cu) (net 4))
 (segment (start 142.75654 100.2628) (end 143.03994 99.9794) (width 0.25) (layer F.Cu) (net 4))
 (segment (start 143.03994 99.9794) (end 144.40164 99.9794) (width 0.25) (layer F.Cu) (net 4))
 (segment (start 139.44794 103.5714) (end 142.75654 100.2628) (width 0.25) (layer F.Cu) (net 4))
 (segment (start 139.44794 96.9543) (end 142.75654 100.2628) (width 0.25) (layer F.Cu) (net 4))
 (segment (start 159.80194 101.7244) (end 159.80194 101.0586) (width 0.25) (layer F.Cu) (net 5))
 (segment (start 159.80194 101.0586) (end 161.38144 99.4791) (width 0.25) (layer F.Cu) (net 5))
 (segment (start 137.79794 103.5714) (end 139.41044 101.9589) (width 0.25) (layer F.Cu) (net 6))
 (segment (start 139.41044 101.9589) (end 139.41044 101.4552) (width 0.25) (layer F.Cu) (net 6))
 (segment (start 136.57754 102.2628) (end 137.02784 102.2628) (width 0.25) (layer F.Cu) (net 7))
 (segment (start 137.02784 102.2628) (end 137.83544 101.4552) (width 0.25) (layer F.Cu) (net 7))
 (segment (start 134.81224 101.5264) (end 135.54864 102.2628) (width 0.25) (layer F.Cu) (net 7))
 (segment (start 135.54864 102.2628) (end 136.57754 102.2628) (width 0.25) (layer F.Cu) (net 7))
 (segment (start 136.57754 102.2628) (end 136.57754 104.2642) (width 0.25) (layer F.Cu) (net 7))
 (segment (start 136.57754 104.2642) (end 138.42474 106.1114) (width 0.25) (layer F.Cu) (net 7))
 (segment (start 138.42474 106.1114) (end 144.94794 106.1114) (width 0.25) (layer F.Cu) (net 7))
 (segment (start 133.63694 101.5264) (end 134.81224 101.5264) (width 0.25) (layer F.Cu) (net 7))
 (segment (start 137.79794 96.9543) (end 139.41044 98.5668) (width 0.25) (layer F.Cu) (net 9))
 (segment (start 139.41044 98.5668) (end 139.41044 99.0142) (width 0.25) (layer F.Cu) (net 9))
 (segment (start 137.83544 99.0142) (end 134.84004 99.0142) (width 0.25) (layer F.Cu) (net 8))
 (segment (start 134.84004 99.0142) (end 134.81224 98.9864) (width 0.25) (layer F.Cu) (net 8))
 (segment (start 144.89494 104.5384) (end 137.48864 104.5384) (width 0.25) (layer F.Cu) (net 8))
 (segment (start 137.48864 104.5384) (end 137.02784 104.0776) (width 0.25) (layer F.Cu) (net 8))
 (segment (start 137.02784 104.0776) (end 137.02784 103.1128) (width 0.25) (layer F.Cu) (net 8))
 (segment (start 137.02784 103.1128) (end 137.88064 102.26) (width 0.25) (layer F.Cu) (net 8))
 (segment (start 137.88064 102.26) (end 138.32444 102.26) (width 0.25) (layer F.Cu) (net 8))
 (segment (start 138.32444 102.26) (end 138.62294 101.9615) (width 0.25) (layer F.Cu) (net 8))
 (segment (start 138.62294 101.9615) (end 138.62294 99.8017) (width 0.25) (layer F.Cu) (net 8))
 (segment (start 138.62294 99.8017) (end 137.83544 99.0142) (width 0.25) (layer F.Cu) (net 8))
 (segment (start 133.63694 98.9864) (end 134.81224 98.9864) (width 0.25) (layer F.Cu) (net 8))
 (segment (start 145.57694 97.4394) (end 144.40164 97.4394) (width 0.25) (layer B.Cu) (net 12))
 (segment (start 144.40164 97.4394) (end 137.77464 104.0664) (width 0.25) (layer B.Cu) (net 12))
 (segment (start 137.77464 104.0664) (end 133.63694 104.0664) (width 0.25) (layer B.Cu) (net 12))
 (segment (start 145.96794 106.1114) (end 147.34534 104.734) (width 0.25) (layer F.Cu) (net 13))
 (segment (start 147.34534 104.734) (end 147.34534 102.1933) (width 0.25) (layer F.Cu) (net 13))
 (segment (start 147.34534 102.1933) (end 150.46824 99.0704) (width 0.25) (layer F.Cu) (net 13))
 (segment (start 150.46824 99.0704) (end 150.87494 99.0704) (width 0.25) (layer F.Cu) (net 13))
 (segment (start 150.87494 100.3404) (end 151.31324 100.3404) (width 0.25) (layer F.Cu) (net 14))
 (segment (start 151.31324 100.3404) (end 152.18484 99.4688) (width 0.25) (layer F.Cu) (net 14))
 (segment (start 152.18484 99.4688) (end 152.18484 98.7241) (width 0.25) (layer F.Cu) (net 14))
 (segment (start 152.18484 98.7241) (end 151.89614 98.4354) (width 0.25) (layer F.Cu) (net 14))
 (segment (start 151.89614 98.4354) (end 149.84934 98.4354) (width 0.25) (layer F.Cu) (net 14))
 (segment (start 149.84934 98.4354) (end 145.91494 102.3698) (width 0.25) (layer F.Cu) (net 14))
 (segment (start 145.91494 102.3698) (end 145.91494 104.5384) (width 0.25) (layer F.Cu) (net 14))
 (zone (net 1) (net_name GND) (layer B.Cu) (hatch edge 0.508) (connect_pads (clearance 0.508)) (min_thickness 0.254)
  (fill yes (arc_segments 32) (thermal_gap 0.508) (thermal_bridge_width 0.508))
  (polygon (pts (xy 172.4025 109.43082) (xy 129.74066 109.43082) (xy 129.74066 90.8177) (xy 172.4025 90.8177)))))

